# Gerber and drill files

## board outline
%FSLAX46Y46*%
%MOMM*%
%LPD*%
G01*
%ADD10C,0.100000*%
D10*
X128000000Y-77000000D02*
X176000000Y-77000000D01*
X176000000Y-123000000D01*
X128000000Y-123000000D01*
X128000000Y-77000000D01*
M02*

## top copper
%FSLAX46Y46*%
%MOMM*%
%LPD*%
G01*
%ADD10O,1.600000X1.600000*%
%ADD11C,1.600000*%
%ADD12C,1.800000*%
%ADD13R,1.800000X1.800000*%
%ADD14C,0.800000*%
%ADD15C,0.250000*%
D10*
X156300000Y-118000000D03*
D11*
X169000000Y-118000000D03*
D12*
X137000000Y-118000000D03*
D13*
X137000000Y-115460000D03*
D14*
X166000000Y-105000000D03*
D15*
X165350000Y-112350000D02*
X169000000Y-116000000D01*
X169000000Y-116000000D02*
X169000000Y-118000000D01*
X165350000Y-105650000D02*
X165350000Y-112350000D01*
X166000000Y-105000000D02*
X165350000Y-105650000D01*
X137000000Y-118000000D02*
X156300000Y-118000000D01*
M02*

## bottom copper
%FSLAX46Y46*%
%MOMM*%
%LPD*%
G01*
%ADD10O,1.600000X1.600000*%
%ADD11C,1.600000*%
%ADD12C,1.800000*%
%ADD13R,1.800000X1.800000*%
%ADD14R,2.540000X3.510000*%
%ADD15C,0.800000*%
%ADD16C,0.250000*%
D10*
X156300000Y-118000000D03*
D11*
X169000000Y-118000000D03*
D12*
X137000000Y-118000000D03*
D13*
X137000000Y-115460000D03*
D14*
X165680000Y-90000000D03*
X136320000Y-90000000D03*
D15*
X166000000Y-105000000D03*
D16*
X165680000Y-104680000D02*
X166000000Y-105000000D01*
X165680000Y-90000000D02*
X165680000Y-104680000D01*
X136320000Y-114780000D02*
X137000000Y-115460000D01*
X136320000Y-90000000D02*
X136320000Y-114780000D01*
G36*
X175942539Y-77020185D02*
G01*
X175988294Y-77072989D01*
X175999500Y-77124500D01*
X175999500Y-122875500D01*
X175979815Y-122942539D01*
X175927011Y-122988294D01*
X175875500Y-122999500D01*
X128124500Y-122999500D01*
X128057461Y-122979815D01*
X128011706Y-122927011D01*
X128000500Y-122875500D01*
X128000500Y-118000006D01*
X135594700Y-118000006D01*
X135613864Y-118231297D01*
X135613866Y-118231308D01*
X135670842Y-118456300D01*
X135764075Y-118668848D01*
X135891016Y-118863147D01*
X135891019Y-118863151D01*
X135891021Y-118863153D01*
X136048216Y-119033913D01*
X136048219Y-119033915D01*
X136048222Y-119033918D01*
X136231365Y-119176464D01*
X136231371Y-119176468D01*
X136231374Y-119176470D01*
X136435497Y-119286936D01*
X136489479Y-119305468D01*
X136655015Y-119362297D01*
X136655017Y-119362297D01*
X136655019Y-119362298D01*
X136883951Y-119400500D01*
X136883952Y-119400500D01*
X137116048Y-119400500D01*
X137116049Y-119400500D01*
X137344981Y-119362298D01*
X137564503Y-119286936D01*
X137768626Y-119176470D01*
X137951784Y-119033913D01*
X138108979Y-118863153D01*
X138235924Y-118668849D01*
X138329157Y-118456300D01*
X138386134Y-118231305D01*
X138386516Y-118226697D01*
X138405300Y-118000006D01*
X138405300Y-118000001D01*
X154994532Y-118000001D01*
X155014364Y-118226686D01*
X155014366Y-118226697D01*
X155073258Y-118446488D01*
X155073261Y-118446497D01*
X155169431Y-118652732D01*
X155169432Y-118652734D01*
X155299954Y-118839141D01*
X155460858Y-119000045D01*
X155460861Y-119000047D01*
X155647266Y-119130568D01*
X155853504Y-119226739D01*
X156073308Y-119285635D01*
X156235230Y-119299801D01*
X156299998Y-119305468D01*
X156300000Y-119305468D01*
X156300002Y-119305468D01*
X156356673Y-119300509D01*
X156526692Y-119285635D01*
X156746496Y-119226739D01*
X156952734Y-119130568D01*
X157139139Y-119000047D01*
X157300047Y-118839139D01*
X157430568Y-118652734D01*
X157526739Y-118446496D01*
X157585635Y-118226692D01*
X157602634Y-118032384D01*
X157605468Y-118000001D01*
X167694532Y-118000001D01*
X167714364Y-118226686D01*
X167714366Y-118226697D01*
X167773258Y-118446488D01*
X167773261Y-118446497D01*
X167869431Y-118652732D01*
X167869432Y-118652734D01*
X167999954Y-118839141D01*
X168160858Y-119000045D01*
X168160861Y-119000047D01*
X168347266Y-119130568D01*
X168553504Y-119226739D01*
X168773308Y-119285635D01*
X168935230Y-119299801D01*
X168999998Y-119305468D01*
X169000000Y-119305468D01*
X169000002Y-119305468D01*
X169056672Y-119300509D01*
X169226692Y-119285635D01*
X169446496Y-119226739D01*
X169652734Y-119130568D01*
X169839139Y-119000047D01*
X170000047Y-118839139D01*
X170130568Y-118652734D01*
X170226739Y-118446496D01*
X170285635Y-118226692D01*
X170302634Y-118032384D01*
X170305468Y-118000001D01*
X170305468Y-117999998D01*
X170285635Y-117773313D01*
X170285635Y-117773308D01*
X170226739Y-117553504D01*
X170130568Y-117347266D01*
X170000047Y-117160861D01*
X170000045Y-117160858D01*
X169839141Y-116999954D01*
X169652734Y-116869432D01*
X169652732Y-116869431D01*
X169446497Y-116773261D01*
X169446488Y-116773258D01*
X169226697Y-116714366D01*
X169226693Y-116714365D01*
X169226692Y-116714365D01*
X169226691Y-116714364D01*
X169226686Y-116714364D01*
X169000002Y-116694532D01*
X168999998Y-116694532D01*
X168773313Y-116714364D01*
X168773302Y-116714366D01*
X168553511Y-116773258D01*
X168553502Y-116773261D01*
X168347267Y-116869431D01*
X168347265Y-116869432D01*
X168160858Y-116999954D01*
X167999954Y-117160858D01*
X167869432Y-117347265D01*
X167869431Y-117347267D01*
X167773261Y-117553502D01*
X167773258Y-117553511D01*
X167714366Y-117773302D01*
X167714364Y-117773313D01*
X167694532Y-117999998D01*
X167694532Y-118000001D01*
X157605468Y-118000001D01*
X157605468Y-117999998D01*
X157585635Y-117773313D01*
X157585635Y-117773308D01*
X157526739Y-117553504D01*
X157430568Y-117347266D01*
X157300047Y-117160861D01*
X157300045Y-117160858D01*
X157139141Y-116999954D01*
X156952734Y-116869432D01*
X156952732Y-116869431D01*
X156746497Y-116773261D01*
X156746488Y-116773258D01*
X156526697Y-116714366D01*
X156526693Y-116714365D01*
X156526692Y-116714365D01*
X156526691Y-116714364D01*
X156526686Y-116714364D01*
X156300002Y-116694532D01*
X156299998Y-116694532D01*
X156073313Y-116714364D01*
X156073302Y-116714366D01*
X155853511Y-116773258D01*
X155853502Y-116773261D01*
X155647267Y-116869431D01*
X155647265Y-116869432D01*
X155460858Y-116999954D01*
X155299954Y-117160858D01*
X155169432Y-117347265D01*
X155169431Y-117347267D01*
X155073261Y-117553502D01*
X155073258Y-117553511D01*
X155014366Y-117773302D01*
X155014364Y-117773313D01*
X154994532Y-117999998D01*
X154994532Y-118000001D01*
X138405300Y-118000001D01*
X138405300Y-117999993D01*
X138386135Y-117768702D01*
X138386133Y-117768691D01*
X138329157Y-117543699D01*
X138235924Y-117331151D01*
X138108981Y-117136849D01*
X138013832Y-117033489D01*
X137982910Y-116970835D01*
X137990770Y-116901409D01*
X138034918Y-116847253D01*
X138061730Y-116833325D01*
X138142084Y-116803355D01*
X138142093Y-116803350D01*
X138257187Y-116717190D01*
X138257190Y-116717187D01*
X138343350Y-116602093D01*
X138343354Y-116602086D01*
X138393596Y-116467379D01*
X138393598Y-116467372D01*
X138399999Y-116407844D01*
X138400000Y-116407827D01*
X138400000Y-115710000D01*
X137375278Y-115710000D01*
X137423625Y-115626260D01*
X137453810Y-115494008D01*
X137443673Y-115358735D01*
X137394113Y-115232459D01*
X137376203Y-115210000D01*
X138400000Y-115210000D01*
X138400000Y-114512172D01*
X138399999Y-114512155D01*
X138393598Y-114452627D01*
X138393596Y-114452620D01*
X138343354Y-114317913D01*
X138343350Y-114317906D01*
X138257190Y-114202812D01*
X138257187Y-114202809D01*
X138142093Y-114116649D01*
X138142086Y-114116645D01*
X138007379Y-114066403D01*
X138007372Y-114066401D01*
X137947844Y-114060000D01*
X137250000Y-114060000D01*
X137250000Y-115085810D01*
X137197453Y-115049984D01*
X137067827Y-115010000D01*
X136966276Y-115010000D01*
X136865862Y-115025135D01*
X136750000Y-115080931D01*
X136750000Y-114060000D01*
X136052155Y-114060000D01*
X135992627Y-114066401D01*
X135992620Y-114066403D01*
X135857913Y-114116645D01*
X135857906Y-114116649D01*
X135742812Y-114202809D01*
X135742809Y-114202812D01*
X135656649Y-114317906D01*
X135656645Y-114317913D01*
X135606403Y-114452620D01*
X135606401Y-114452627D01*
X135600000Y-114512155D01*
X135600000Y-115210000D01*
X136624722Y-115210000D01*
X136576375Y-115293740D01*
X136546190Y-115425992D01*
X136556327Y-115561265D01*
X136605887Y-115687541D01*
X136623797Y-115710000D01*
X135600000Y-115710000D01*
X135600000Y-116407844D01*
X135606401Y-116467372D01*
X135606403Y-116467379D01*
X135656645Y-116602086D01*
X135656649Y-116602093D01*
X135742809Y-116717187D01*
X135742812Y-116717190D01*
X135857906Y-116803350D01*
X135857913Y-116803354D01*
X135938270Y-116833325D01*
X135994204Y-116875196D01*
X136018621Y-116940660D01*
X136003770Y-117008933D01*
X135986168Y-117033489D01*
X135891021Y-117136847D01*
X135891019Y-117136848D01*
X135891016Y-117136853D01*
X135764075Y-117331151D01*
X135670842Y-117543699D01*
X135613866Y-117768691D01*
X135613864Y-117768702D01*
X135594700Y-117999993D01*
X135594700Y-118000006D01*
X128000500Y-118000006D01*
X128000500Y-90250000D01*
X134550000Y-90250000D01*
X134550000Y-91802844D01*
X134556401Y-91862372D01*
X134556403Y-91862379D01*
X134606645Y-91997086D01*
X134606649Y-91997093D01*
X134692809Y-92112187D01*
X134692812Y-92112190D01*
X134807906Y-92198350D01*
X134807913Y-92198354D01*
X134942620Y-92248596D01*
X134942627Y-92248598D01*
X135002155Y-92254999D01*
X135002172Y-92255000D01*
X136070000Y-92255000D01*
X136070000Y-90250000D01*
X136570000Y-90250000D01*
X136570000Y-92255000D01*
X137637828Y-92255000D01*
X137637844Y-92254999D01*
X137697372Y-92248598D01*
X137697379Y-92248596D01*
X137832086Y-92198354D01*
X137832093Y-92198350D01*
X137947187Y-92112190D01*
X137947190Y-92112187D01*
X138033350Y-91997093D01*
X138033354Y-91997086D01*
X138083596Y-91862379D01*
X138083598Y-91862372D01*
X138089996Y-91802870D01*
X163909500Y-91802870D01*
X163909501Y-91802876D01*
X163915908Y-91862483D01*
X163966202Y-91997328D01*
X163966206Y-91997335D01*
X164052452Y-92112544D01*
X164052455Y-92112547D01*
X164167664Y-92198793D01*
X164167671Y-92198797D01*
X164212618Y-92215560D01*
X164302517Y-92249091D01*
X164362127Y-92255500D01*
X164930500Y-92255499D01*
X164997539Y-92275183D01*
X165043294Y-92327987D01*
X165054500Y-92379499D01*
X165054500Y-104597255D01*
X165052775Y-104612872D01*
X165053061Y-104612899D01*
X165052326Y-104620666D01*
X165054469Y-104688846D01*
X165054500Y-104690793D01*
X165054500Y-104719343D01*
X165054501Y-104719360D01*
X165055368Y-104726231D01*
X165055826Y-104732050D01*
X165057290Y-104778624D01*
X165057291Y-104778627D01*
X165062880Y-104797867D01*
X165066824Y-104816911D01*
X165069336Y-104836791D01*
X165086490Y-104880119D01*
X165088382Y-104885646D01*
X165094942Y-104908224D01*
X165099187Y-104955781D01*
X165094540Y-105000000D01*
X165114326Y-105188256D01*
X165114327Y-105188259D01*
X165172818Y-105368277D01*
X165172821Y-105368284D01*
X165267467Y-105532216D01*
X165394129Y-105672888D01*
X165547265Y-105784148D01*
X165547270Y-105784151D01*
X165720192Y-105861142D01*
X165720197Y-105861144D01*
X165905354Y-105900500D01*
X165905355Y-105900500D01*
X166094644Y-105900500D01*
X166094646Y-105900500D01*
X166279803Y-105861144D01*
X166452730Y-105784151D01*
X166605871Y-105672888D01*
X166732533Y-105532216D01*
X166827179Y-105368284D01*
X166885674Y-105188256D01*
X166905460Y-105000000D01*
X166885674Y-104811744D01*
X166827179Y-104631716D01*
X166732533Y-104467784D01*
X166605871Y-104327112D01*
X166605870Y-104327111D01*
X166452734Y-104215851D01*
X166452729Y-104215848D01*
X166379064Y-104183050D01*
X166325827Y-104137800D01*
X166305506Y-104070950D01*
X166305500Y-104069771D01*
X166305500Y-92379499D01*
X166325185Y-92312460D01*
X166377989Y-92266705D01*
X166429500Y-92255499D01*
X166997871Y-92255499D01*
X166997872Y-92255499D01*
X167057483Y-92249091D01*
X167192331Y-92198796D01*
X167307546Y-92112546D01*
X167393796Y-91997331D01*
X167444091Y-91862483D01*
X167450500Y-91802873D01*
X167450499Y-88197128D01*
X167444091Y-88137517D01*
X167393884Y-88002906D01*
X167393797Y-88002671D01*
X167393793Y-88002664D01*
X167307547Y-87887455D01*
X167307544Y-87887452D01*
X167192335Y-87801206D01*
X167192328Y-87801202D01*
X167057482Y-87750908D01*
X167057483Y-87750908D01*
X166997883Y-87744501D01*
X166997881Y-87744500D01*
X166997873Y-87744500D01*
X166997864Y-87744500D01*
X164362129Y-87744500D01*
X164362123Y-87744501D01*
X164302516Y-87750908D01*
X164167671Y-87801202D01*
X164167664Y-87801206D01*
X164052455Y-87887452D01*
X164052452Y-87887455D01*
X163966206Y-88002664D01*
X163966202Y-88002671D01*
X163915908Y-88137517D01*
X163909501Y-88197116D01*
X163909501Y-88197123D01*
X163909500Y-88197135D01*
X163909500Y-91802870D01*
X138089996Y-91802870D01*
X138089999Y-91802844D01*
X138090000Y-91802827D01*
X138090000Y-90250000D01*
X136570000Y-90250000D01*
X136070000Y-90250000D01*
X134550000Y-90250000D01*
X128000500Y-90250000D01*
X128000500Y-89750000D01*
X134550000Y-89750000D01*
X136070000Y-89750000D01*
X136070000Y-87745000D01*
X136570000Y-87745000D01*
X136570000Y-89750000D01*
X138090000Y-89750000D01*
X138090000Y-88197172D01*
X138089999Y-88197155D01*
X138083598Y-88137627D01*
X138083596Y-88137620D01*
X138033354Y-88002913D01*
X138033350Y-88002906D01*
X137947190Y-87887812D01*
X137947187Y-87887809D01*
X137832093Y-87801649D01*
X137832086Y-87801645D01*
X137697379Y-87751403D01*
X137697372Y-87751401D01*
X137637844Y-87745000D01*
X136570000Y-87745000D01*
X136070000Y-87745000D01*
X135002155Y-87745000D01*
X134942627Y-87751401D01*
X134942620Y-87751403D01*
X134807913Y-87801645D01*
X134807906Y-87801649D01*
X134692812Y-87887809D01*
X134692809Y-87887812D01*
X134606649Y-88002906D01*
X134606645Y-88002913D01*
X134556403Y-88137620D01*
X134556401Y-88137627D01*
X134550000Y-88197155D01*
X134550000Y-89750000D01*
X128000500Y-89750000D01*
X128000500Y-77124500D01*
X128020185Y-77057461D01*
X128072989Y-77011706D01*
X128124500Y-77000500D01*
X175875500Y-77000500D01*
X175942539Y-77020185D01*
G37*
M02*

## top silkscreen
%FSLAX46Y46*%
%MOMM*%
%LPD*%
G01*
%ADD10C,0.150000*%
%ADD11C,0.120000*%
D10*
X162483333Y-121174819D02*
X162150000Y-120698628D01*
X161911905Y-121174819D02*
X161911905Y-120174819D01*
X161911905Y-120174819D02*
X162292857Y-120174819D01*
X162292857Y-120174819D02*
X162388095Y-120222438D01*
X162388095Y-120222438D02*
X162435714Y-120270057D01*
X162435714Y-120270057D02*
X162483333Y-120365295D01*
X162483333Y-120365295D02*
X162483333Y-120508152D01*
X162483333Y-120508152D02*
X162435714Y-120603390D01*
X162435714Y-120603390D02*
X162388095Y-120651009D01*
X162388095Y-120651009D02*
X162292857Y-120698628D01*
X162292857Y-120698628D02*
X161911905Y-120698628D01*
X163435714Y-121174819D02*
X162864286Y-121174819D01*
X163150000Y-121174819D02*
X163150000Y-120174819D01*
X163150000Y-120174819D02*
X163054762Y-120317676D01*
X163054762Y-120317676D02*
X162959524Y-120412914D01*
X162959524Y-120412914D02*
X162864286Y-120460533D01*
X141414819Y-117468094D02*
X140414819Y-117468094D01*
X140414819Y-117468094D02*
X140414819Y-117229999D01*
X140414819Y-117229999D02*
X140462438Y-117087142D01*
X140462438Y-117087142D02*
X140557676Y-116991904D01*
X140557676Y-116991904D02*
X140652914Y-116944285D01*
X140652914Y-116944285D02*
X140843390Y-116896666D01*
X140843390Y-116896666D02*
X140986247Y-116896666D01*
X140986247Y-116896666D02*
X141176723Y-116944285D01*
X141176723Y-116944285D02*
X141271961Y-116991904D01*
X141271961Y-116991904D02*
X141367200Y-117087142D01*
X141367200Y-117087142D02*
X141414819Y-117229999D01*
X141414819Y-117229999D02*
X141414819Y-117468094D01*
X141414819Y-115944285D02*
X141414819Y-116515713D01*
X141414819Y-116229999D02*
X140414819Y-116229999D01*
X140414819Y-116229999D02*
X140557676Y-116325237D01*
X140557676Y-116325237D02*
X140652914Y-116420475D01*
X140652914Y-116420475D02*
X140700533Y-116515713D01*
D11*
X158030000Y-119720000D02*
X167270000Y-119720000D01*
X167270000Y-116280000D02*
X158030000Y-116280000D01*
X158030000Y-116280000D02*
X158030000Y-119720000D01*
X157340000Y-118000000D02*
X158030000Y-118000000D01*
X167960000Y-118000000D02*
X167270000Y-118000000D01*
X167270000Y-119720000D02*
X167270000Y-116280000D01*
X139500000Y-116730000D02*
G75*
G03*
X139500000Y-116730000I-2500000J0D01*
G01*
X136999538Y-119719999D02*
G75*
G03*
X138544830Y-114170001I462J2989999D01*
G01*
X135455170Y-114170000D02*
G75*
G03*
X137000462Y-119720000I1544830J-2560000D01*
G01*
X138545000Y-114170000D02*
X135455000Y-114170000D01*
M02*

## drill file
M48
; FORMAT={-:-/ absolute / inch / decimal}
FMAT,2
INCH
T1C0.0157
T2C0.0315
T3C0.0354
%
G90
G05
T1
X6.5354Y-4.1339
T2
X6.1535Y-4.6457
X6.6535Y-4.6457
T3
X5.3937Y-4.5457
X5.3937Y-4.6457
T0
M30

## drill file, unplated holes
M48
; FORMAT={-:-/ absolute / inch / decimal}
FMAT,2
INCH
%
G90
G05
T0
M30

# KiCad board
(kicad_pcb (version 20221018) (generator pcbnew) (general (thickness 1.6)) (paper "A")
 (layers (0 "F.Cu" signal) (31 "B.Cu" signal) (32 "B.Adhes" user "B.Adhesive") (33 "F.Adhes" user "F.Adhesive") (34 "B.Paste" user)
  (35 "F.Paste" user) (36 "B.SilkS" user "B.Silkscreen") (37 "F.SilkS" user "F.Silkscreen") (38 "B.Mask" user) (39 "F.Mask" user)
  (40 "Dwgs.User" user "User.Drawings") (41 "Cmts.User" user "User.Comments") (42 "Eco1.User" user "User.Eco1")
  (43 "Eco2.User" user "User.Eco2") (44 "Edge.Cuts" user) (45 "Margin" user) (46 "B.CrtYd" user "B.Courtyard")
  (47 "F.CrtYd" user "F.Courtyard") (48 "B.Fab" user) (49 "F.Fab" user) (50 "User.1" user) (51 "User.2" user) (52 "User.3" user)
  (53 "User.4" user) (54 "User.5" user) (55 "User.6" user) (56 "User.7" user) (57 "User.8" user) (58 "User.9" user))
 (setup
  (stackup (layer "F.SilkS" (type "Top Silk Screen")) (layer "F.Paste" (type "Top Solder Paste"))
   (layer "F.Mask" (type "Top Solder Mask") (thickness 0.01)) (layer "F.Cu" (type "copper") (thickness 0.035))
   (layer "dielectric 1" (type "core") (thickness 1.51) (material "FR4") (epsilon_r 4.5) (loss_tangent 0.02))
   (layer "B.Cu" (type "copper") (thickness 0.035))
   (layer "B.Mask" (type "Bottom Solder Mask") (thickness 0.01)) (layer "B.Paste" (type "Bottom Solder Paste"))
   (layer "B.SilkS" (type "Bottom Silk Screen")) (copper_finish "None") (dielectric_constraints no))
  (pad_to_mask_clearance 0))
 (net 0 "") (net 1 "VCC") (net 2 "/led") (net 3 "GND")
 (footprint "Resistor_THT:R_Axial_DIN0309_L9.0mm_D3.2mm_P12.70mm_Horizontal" (layer "F.Cu") (at 169 118 180)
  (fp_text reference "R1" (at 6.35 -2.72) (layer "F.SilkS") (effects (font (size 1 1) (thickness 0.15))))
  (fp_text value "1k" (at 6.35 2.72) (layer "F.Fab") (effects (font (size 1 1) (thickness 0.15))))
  (fp_line (start 1.04 0) (end 1.73 0) (stroke (width 0.12) (type solid)) (layer "F.SilkS"))
  (fp_line (start 1.73 -1.72) (end 1.73 1.72) (stroke (width 0.12) (type solid)) (layer "F.SilkS"))
  (fp_line (start 1.73 1.72) (end 10.97 1.72) (stroke (width 0.12) (type solid)) (layer "F.SilkS"))
  (fp_line (start 10.97 -1.72) (end 1.73 -1.72) (stroke (width 0.12) (type solid)) (layer "F.SilkS"))
  (fp_line (start 10.97 1.72) (end 10.97 -1.72) (stroke (width 0.12) (type solid)) (layer "F.SilkS"))
  (fp_line (start 11.66 0) (end 10.97 0) (stroke (width 0.12) (type solid)) (layer "F.SilkS"))
  (pad "1" thru_hole circle (at 0 0 180) (size 1.6 1.6) (drill 0.8) (layers "*.Cu" "*.Mask") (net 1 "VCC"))
  (pad "2" thru_hole oval (at 12.7 0 180) (size 1.6 1.6) (drill 0.8) (layers "*.Cu" "*.Mask") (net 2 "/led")))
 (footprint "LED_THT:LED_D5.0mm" (layer "F.Cu") (at 137 115.46 -90)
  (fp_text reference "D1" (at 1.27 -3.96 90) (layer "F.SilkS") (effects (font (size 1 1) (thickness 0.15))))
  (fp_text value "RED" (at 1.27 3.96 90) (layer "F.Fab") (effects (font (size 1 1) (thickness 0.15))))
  (fp_line (start -1.29 -1.545) (end -1.29 1.545) (stroke (width 0.12) (type solid)) (layer "F.SilkS"))
  (fp_arc (start -1.29 -1.54483) (mid 2.072002 -2.880433) (end 4.26 0.000462) (stroke (width 0.12) (type solid)) (layer "F.SilkS"))
  (fp_arc (start 4.26 -0.000462) (mid 2.072002 2.880433) (end -1.29 1.54483) (stroke (width 0.12) (type solid)) (layer "F.SilkS"))
  (fp_circle (center 1.27 0) (end 3.77 0) (stroke (width 0.12) (type solid)) (fill none) (layer "F.SilkS"))
  (pad "1" thru_hole rect (at 0 0 270) (size 1.8 1.8) (drill 0.9) (layers "*.Cu" "*.Mask") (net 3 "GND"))
  (pad "2" thru_hole circle (at 2.54 0 270) (size 1.8 1.8) (drill 0.9) (layers "*.Cu" "*.Mask") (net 2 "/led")))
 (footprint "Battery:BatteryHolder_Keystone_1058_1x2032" (layer "B.Cu") (at 151 90 180)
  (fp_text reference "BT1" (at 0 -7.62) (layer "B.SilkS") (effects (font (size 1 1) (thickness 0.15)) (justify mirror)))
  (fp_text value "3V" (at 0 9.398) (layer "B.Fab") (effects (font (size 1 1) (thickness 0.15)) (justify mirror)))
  (pad "1" smd rect (at -14.68 0 180) (size 2.54 3.51) (layers "B.Cu" "B.Paste" "B.Mask") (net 1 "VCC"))
  (pad "2" smd rect (at 14.68 0 180) (size 2.54 3.51) (layers "B.Cu" "B.Paste" "B.Mask") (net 3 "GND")))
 (gr_rect (start 128 77) (end 176 123) (stroke (width 0.1) (type default)) (fill none) (layer "Edge.Cuts"))
 (segment (start 165.35 105.65) (end 165.35 112.35) (width 0.25) (layer "F.Cu") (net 1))
 (segment (start 166 105) (end 165.35 105.65) (width 0.25) (layer "F.Cu") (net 1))
 (segment (start 169 116) (end 169 118) (width 0.25) (layer "F.Cu") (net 1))
 (segment (start 165.35 112.35) (end 169 116) (width 0.25) (layer "F.Cu") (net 1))
 (via (at 166 105) (size 0.8) (drill 0.4) (layers "F.Cu" "B.Cu") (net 1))
 (segment (start 165.68 104.68) (end 166 105) (width 0.25) (layer "B.Cu") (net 1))
 (segment (start 165.68 90) (end 165.68 104.68) (width 0.25) (layer "B.Cu") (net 1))
 (segment (start 136.32 114.78) (end 137 115.46) (width 0.25) (layer "B.Cu") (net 3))
 (segment (start 136.32 90) (end 136.32 114.78) (width 0.25) (layer "B.Cu") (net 3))
 (segment (start 137 118) (end 156.3 118) (width 0.25) (layer "F.Cu") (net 2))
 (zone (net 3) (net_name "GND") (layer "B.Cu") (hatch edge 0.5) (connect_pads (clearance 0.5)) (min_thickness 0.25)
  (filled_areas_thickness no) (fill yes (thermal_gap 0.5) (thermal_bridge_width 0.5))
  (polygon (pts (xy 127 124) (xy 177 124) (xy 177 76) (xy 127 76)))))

